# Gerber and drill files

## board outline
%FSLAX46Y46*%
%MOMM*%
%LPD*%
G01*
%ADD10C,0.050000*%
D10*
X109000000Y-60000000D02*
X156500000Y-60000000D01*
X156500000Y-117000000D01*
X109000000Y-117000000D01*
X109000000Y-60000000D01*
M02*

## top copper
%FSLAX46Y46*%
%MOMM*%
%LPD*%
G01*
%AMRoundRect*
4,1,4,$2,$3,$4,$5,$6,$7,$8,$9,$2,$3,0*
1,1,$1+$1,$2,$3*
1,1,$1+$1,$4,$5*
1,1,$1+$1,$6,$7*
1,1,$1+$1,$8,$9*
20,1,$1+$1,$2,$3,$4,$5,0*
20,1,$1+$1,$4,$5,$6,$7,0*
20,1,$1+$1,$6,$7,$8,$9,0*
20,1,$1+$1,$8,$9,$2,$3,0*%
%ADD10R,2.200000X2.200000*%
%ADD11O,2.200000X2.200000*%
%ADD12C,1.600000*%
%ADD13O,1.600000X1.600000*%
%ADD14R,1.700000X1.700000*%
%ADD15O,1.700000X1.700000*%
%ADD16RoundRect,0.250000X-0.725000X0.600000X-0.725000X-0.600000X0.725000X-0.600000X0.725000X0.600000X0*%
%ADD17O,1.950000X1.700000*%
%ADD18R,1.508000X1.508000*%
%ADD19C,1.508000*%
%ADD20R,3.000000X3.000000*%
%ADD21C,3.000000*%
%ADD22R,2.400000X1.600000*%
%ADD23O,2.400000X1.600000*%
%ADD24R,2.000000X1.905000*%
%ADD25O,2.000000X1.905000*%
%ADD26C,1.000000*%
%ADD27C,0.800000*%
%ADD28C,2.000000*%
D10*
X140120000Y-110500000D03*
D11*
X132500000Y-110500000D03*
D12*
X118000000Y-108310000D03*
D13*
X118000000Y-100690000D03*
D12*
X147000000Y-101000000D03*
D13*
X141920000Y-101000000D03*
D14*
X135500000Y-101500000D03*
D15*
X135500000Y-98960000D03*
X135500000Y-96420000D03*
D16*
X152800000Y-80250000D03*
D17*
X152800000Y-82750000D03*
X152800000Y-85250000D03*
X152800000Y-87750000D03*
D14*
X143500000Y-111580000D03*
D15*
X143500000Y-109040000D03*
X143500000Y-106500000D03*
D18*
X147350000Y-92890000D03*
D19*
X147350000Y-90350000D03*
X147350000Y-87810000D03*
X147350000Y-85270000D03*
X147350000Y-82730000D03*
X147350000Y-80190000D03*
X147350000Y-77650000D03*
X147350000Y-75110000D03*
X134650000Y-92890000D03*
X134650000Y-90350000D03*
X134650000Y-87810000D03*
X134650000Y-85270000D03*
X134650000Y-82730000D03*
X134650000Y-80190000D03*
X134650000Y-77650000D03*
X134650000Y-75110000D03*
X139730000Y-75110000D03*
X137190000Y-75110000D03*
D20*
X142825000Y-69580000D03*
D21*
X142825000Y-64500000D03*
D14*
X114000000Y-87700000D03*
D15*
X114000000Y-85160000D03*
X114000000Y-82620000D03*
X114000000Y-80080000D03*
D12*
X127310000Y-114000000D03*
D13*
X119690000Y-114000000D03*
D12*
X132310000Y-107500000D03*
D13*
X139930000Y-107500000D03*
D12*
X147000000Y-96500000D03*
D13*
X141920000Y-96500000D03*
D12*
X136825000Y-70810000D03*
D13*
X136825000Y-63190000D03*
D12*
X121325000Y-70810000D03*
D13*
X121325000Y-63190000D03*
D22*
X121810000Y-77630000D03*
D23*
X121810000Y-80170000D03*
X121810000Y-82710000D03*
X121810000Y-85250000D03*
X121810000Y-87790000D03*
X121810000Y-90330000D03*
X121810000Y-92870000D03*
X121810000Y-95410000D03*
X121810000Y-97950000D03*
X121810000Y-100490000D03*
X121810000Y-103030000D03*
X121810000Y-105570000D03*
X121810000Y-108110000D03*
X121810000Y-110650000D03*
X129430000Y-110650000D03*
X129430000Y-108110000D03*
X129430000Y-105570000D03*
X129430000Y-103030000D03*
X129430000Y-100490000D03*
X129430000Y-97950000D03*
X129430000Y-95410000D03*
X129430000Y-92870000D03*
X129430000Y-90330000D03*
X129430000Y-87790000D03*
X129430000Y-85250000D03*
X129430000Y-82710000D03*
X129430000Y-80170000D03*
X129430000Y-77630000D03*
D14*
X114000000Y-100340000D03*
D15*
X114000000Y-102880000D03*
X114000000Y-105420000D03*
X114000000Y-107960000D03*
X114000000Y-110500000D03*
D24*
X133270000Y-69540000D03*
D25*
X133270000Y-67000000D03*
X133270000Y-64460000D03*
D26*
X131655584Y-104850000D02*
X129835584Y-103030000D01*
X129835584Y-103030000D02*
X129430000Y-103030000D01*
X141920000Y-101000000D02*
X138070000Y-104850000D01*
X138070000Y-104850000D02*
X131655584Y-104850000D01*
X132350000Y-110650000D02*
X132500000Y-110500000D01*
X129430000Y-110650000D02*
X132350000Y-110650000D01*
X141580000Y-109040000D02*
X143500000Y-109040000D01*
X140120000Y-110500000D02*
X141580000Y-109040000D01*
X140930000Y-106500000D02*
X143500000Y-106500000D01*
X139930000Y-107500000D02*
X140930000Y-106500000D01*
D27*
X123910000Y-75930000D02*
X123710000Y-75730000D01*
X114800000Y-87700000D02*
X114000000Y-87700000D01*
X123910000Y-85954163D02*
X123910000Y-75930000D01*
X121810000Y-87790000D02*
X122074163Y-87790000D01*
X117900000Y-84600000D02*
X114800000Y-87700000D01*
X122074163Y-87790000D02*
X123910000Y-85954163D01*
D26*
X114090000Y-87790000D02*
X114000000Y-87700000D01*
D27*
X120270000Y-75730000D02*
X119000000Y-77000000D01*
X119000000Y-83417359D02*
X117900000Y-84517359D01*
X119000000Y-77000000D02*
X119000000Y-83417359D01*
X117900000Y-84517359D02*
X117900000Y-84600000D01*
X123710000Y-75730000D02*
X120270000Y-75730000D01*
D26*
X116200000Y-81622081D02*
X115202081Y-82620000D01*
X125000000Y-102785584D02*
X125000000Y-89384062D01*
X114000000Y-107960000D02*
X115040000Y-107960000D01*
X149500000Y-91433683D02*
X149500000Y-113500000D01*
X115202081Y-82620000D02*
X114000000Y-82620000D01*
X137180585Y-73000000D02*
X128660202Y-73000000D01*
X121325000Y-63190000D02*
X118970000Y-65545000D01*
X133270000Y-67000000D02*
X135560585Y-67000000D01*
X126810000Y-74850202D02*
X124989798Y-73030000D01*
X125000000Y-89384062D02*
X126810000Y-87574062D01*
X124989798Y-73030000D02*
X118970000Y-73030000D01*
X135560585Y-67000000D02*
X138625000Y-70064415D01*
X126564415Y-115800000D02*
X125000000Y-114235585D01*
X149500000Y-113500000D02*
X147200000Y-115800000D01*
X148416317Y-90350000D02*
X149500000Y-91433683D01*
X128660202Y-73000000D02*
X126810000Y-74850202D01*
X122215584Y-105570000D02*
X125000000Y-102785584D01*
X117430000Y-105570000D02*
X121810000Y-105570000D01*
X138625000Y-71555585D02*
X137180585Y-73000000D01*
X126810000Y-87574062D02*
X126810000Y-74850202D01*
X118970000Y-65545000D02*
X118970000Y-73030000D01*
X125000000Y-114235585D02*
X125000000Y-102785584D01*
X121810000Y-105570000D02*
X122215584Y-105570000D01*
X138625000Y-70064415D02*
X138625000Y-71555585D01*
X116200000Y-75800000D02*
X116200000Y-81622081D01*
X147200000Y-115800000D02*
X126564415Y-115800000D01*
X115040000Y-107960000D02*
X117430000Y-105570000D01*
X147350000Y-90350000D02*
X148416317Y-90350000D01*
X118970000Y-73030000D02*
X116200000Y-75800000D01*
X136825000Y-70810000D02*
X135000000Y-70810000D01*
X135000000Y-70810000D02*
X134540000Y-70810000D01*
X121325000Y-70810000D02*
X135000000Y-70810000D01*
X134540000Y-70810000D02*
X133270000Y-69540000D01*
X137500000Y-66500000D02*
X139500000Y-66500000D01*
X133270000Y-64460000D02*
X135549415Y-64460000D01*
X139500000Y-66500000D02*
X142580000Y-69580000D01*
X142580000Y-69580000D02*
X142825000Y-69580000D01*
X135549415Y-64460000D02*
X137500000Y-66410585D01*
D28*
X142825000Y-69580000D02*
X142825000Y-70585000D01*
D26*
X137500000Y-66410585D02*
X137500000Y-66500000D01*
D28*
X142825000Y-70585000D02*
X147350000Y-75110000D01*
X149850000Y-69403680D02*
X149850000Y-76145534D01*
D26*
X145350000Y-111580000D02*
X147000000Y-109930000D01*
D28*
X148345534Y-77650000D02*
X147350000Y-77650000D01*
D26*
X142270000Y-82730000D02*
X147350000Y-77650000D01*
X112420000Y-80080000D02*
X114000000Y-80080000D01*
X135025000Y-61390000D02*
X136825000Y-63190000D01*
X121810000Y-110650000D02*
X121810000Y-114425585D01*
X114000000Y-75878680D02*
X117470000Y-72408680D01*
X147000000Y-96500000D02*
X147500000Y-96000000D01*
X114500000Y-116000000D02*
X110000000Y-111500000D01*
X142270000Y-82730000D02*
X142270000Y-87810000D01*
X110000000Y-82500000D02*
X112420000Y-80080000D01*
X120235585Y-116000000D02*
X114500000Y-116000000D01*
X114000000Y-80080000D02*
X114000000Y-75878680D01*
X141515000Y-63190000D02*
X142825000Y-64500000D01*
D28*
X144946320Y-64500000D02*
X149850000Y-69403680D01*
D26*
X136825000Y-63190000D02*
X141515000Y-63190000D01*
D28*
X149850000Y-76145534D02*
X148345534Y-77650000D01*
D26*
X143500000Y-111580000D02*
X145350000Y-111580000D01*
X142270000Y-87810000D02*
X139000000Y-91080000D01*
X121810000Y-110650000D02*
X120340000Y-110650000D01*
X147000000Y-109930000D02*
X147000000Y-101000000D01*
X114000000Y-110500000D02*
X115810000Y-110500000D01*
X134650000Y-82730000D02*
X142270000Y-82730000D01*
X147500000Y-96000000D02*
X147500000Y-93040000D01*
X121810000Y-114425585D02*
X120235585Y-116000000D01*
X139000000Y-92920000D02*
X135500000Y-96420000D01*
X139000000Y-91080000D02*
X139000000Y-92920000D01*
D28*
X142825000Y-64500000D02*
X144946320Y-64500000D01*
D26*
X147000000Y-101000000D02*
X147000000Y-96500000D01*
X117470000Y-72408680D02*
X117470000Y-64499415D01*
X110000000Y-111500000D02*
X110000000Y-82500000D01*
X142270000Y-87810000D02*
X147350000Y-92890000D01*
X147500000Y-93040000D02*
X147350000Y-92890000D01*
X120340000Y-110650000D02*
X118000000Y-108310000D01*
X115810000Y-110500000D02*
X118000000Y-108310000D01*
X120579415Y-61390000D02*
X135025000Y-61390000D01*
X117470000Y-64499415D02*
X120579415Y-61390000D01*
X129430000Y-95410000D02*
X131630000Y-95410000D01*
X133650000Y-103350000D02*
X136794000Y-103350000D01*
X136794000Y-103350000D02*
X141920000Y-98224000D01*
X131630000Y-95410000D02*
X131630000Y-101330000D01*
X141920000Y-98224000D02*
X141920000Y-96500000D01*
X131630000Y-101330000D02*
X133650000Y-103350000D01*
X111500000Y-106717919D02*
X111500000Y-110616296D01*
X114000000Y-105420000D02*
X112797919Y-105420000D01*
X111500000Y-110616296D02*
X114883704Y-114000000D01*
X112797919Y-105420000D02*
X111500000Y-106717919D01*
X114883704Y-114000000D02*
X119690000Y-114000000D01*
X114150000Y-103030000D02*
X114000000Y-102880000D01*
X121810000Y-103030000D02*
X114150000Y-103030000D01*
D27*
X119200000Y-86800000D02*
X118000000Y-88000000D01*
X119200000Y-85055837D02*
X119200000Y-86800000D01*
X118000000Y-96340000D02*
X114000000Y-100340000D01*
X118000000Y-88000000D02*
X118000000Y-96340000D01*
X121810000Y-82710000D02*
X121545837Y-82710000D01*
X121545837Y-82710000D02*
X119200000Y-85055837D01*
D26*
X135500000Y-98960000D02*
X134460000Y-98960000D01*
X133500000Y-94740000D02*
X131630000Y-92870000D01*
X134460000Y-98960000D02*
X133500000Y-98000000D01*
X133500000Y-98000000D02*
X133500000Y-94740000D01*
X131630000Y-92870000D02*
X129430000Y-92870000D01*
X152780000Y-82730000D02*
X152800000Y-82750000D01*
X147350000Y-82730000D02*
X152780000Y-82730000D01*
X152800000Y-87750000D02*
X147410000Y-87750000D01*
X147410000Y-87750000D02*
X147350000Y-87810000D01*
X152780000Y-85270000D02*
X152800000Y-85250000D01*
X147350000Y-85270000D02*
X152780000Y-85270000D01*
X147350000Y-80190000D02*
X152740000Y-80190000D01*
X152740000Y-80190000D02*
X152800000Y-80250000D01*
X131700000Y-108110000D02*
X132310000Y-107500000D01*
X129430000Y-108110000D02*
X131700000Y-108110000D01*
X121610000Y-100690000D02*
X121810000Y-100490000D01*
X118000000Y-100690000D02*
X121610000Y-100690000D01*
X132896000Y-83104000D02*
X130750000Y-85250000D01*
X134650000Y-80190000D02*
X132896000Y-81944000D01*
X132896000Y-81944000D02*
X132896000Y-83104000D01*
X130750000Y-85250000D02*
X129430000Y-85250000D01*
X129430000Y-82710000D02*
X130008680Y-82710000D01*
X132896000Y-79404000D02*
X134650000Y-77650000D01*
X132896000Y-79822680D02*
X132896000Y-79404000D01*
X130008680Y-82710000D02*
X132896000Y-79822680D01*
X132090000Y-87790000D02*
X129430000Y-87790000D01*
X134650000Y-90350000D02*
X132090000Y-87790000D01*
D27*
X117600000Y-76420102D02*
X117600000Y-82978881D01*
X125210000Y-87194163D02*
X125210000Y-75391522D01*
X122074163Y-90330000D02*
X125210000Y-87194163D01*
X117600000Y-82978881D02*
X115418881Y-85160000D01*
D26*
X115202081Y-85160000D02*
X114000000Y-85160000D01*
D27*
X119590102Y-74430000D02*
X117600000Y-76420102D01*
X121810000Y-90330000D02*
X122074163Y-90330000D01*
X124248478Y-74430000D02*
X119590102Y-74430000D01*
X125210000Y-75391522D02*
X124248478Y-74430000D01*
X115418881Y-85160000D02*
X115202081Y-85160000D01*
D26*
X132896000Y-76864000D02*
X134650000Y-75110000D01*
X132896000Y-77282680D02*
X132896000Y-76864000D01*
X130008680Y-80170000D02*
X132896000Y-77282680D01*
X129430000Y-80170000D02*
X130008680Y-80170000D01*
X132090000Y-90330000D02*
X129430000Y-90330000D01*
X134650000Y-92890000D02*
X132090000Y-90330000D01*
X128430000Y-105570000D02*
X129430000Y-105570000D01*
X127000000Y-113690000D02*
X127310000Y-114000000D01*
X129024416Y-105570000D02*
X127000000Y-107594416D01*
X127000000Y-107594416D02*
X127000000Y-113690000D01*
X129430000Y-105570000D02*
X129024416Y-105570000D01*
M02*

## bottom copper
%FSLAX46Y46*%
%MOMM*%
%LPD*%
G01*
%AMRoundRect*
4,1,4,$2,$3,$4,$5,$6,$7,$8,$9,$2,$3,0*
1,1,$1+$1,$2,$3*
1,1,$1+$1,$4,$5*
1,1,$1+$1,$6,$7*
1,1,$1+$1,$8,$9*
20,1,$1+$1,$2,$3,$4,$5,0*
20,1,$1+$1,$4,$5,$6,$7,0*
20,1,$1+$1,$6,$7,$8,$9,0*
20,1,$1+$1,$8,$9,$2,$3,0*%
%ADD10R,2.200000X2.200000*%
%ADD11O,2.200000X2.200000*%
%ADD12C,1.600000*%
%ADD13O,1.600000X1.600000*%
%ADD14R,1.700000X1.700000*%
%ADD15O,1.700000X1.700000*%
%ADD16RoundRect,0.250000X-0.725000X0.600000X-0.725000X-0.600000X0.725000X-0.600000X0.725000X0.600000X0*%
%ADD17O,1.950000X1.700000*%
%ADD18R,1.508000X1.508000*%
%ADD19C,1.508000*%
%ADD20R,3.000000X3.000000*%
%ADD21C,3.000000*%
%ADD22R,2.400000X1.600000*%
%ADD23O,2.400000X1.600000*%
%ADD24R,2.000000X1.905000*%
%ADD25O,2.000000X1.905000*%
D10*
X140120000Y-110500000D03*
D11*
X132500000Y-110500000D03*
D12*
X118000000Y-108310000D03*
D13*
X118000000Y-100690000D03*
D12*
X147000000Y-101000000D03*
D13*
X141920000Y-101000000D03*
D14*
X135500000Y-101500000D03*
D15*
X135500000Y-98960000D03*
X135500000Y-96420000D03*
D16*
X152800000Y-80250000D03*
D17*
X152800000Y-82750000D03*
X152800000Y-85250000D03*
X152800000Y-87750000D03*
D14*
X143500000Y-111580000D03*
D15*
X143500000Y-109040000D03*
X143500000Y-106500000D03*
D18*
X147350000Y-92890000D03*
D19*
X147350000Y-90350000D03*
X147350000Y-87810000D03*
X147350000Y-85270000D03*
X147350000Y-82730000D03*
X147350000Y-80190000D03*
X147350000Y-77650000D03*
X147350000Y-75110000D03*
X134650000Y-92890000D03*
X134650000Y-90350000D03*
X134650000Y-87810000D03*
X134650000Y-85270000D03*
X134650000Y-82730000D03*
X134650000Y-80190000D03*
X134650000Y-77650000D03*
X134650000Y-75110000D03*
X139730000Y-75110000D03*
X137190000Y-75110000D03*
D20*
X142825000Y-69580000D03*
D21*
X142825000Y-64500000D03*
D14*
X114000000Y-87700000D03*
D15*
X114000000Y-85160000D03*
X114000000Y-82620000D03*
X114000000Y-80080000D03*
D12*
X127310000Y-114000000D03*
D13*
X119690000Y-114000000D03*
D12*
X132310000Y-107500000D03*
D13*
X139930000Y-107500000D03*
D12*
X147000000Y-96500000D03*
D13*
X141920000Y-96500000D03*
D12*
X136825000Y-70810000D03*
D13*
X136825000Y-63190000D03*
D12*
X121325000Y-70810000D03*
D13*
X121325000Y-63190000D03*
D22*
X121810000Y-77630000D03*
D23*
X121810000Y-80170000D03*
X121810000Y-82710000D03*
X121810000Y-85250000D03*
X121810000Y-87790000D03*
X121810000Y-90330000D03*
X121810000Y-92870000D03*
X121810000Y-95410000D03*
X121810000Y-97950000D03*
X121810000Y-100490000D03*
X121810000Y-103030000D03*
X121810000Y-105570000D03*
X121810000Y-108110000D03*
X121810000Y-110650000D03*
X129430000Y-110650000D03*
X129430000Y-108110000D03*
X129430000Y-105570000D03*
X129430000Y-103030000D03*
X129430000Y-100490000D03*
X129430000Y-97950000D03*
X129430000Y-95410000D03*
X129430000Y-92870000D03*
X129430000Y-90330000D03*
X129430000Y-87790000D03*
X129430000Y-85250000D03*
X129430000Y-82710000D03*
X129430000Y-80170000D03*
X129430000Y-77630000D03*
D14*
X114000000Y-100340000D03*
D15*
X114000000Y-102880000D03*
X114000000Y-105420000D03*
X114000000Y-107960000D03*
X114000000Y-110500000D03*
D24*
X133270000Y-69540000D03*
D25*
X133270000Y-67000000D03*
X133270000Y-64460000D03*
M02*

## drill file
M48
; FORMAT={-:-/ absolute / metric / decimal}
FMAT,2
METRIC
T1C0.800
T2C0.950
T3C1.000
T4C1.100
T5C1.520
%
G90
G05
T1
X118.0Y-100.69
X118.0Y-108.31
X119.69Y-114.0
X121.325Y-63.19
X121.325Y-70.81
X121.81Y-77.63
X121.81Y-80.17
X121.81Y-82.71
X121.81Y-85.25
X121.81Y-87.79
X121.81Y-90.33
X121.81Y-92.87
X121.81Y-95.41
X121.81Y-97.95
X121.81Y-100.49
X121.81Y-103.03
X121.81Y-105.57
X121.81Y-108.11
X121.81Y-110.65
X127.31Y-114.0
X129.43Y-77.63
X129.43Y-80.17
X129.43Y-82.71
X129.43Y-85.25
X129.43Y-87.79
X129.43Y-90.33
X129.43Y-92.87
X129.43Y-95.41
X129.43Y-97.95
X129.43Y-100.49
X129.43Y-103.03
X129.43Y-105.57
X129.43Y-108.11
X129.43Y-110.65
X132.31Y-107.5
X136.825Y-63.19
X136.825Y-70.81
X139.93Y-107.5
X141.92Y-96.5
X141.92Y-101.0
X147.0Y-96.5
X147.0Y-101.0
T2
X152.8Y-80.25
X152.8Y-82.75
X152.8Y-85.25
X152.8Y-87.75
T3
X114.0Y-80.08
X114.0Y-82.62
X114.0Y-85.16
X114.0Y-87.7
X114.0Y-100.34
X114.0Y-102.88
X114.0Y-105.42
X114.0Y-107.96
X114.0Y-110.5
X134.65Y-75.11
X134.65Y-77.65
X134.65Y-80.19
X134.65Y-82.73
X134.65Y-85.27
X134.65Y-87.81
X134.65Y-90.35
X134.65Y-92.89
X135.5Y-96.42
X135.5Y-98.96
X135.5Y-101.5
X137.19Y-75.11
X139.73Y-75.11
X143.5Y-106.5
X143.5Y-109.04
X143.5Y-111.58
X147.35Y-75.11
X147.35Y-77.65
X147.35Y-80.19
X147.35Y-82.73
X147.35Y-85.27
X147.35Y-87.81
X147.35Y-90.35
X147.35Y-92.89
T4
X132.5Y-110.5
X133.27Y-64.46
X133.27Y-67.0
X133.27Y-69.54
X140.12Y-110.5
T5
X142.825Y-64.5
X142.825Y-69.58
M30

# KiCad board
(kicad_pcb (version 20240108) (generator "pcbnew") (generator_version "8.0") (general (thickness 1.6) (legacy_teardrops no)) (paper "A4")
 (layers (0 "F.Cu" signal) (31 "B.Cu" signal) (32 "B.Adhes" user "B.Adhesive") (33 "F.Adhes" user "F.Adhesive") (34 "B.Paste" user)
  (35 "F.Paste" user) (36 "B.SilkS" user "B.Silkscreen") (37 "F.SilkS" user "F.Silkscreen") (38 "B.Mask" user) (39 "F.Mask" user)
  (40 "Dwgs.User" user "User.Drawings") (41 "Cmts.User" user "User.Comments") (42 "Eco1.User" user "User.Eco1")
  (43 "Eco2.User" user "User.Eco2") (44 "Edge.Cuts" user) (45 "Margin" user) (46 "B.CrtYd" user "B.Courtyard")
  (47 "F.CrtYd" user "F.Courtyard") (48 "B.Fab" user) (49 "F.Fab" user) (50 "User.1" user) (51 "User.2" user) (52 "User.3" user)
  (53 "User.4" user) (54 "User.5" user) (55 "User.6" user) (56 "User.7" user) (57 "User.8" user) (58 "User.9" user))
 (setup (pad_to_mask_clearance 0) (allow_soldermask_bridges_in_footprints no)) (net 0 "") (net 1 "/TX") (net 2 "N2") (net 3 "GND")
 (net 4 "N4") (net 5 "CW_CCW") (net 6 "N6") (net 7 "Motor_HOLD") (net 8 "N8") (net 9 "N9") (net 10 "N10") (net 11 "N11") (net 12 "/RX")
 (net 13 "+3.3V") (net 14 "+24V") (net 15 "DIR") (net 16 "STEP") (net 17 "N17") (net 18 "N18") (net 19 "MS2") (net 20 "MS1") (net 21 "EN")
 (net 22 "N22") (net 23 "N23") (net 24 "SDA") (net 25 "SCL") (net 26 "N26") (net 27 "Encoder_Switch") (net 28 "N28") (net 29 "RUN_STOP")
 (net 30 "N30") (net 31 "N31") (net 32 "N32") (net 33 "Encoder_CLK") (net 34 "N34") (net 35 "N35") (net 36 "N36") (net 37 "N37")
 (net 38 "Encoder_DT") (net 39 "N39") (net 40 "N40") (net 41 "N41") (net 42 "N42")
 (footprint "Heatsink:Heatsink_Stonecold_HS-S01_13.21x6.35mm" (layer "F.Cu") (at 129.5 67 -90)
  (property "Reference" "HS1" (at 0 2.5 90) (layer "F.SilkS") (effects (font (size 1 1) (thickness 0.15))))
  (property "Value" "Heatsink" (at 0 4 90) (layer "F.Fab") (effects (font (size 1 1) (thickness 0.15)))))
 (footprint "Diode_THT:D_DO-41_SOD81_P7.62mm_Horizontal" (layer "F.Cu") (at 140.12 110.5 180)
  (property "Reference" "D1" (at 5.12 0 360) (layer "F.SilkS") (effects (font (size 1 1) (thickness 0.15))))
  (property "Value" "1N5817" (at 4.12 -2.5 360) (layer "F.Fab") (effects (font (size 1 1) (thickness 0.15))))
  (pad "1" thru_hole rect (at 0 0 180) (size 2.2 2.2) (drill 1.1) (layers "*.Cu" "*.Mask") (remove_unused_layers no) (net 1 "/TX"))
  (pad "2" thru_hole oval (at 7.62 0 180) (size 2.2 2.2) (drill 1.1) (layers "*.Cu" "*.Mask") (remove_unused_layers no) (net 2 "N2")))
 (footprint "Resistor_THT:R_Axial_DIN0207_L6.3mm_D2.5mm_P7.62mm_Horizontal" (layer "F.Cu") (at 118 108.31 90)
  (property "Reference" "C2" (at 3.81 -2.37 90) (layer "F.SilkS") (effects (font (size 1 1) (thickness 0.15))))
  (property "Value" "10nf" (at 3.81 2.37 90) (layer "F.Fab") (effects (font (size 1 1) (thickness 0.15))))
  (pad "1" thru_hole circle (at 0 0 90) (size 1.6 1.6) (drill 0.8) (layers "*.Cu" "*.Mask") (remove_unused_layers no) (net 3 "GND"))
  (pad "2" thru_hole oval (at 7.62 0 90) (size 1.6 1.6) (drill 0.8) (layers "*.Cu" "*.Mask") (remove_unused_layers no) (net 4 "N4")))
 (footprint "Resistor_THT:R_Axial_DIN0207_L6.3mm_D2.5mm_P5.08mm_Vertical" (layer "F.Cu") (at 147 101 180)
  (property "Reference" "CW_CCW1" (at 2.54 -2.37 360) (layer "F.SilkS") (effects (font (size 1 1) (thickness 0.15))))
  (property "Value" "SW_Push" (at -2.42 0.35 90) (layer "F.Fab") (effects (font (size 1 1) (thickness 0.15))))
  (pad "1" thru_hole circle (at 0 0 180) (size 1.6 1.6) (drill 0.8) (layers "*.Cu" "*.Mask") (remove_unused_layers no) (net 3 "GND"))
  (pad "2" thru_hole oval (at 5.08 0 180) (size 1.6 1.6) (drill 0.8) (layers "*.Cu" "*.Mask") (remove_unused_layers no) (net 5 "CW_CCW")))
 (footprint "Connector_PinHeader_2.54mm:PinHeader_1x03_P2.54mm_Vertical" (layer "F.Cu") (at 135.5 101.5 180)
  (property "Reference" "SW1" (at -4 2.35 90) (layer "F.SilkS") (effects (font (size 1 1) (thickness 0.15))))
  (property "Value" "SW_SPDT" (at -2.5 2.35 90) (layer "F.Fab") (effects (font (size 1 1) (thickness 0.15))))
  (pad "1" thru_hole rect (at 0 0 180) (size 1.7 1.7) (drill 1) (layers "*.Cu" "*.Mask") (remove_unused_layers no) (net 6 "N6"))
  (pad "2" thru_hole oval (at 0 2.54 180) (size 1.7 1.7) (drill 1) (layers "*.Cu" "*.Mask") (remove_unused_layers no) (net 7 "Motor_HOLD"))
  (pad "3" thru_hole oval (at 0 5.08 180) (size 1.7 1.7) (drill 1) (layers "*.Cu" "*.Mask") (remove_unused_layers no) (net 3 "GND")))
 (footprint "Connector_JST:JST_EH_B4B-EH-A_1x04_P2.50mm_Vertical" (layer "F.Cu") (at 152.8 80.25 -90)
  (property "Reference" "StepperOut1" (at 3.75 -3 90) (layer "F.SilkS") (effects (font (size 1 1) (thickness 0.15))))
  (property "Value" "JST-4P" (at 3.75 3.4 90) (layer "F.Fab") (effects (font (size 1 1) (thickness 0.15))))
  (pad "1" thru_hole roundrect (at 0 0 270) (size 1.7 1.95) (drill 0.95) (layers "*.Cu" "*.Mask") (remove_unused_layers no)
   (roundrect_rratio 0.147059) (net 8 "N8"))
  (pad "2" thru_hole oval (at 2.5 0 270) (size 1.7 1.95) (drill 0.95) (layers "*.Cu" "*.Mask") (remove_unused_layers no) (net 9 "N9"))
  (pad "3" thru_hole oval (at 5 0 270) (size 1.7 1.95) (drill 0.95) (layers "*.Cu" "*.Mask") (remove_unused_layers no) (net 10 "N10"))
  (pad "4" thru_hole oval (at 7.5 0 270) (size 1.7 1.95) (drill 0.95) (layers "*.Cu" "*.Mask") (remove_unused_layers no) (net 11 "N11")))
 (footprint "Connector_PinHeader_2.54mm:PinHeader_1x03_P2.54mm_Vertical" (layer "F.Cu") (at 143.5 111.58 180)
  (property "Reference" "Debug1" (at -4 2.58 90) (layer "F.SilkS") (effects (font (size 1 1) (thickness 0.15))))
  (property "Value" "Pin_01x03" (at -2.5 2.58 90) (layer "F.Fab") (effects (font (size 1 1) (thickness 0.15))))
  (pad "1" thru_hole rect (at 0 0 180) (size 1.7 1.7) (drill 1) (layers "*.Cu" "*.Mask") (remove_unused_layers no) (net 3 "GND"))
  (pad "2" thru_hole oval (at 0 2.54 180) (size 1.7 1.7) (drill 1) (layers "*.Cu" "*.Mask") (remove_unused_layers no) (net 1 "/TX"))
  (pad "3" thru_hole oval (at 0 5.08 180) (size 1.7 1.7) (drill 1) (layers "*.Cu" "*.Mask") (remove_unused_layers no) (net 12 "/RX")))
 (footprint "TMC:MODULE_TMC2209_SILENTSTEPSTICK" (layer "F.Cu") (at 141 84 180)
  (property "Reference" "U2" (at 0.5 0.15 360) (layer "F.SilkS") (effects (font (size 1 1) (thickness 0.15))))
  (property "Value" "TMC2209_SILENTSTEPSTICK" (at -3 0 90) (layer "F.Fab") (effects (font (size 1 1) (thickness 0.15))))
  (pad "1" thru_hole rect (at -6.35 -8.89 180) (size 1.508 1.508) (drill 1) (layers "*.Cu" "*.Mask") (remove_unused_layers no) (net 3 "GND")
   (solder_mask_margin 0.102))
  (pad "2" thru_hole circle (at -6.35 -6.35 180) (size 1.508 1.508) (drill 1) (layers "*.Cu" "*.Mask") (remove_unused_layers no)
   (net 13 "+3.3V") (solder_mask_margin 0.102))
  (pad "3" thru_hole circle (at -6.35 -3.81 180) (size 1.508 1.508) (drill 1) (layers "*.Cu" "*.Mask") (remove_unused_layers no)
   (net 11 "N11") (solder_mask_margin 0.102))
  (pad "4" thru_hole circle (at -6.35 -1.27 180) (size 1.508 1.508) (drill 1) (layers "*.Cu" "*.Mask") (remove_unused_layers no)
   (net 10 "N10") (solder_mask_margin 0.102))
  (pad "5" thru_hole circle (at -6.35 1.27 180) (size 1.508 1.508) (drill 1) (layers "*.Cu" "*.Mask") (remove_unused_layers no) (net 9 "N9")
   (solder_mask_margin 0.102))
  (pad "6" thru_hole circle (at -6.35 3.81 180) (size 1.508 1.508) (drill 1) (layers "*.Cu" "*.Mask") (remove_unused_layers no) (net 8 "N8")
   (solder_mask_margin 0.102))
  (pad "7" thru_hole circle (at -6.35 6.35 180) (size 1.508 1.508) (drill 1) (layers "*.Cu" "*.Mask") (remove_unused_layers no)
   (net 3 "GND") (solder_mask_margin 0.102))
  (pad "8" thru_hole circle (at -6.35 8.89 180) (size 1.508 1.508) (drill 1) (layers "*.Cu" "*.Mask") (remove_unused_layers no)
   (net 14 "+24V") (solder_mask_margin 0.102))
  (pad "9" thru_hole circle (at 6.35 -8.89 180) (size 1.508 1.508) (drill 1) (layers "*.Cu" "*.Mask") (remove_unused_layers no)
   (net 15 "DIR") (solder_mask_margin 0.102))
  (pad "10" thru_hole circle (at 6.35 -6.35 180) (size 1.508 1.508) (drill 1) (layers "*.Cu" "*.Mask") (remove_unused_layers no)
   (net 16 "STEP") (solder_mask_margin 0.102))
  (pad "11" thru_hole circle (at 6.35 -3.81 180) (size 1.508 1.508) (drill 1) (layers "*.Cu" "*.Mask") (remove_unused_layers no)
   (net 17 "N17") (solder_mask_margin 0.102))
  (pad "12" thru_hole circle (at 6.35 -1.27 180) (size 1.508 1.508) (drill 1) (layers "*.Cu" "*.Mask") (remove_unused_layers no)
   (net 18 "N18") (solder_mask_margin 0.102))
  (pad "13" thru_hole circle (at 6.35 1.27 180) (size 1.508 1.508) (drill 1) (layers "*.Cu" "*.Mask") (remove_unused_layers no)
   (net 3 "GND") (solder_mask_margin 0.102))
  (pad "14" thru_hole circle (at 6.35 3.81 180) (size 1.508 1.508) (drill 1) (layers "*.Cu" "*.Mask") (remove_unused_layers no)
   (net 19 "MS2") (solder_mask_margin 0.102))
  (pad "15" thru_hole circle (at 6.35 6.35 180) (size 1.508 1.508) (drill 1) (layers "*.Cu" "*.Mask") (remove_unused_layers no)
   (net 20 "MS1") (solder_mask_margin 0.102))
  (pad "16" thru_hole circle (at 6.35 8.89 180) (size 1.508 1.508) (drill 1) (layers "*.Cu" "*.Mask") (remove_unused_layers no)
   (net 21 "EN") (solder_mask_margin 0.102))
  (pad "17" thru_hole circle (at 1.27 8.89 180) (size 1.508 1.508) (drill 1) (layers "*.Cu" "*.Mask") (remove_unused_layers no)
   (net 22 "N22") (solder_mask_margin 0.102))
  (pad "18" thru_hole circle (at 3.81 8.89 180) (size 1.508 1.508) (drill 1) (layers "*.Cu" "*.Mask") (remove_unused_layers no)
   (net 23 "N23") (solder_mask_margin 0.102)))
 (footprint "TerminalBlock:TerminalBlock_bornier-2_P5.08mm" (layer "F.Cu") (at 142.825 69.58 90)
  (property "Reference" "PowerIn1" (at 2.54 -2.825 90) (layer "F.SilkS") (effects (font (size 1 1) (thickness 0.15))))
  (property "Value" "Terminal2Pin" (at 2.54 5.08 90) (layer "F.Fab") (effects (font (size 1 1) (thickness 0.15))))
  (pad "1" thru_hole rect (at 0 0 90) (size 3 3) (drill 1.52) (layers "*.Cu" "*.Mask") (remove_unused_layers no) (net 14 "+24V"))
  (pad "2" thru_hole circle (at 5.08 0 90) (size 3 3) (drill 1.52) (layers "*.Cu" "*.Mask") (remove_unused_layers no) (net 3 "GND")))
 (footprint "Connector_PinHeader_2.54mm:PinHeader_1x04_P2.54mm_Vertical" (layer "F.Cu") (at 114 87.7 180)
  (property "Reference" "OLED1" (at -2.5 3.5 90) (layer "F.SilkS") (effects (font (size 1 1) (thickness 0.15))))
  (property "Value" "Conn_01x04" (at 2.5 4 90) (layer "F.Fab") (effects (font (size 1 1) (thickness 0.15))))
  (pad "1" thru_hole rect (at 0 0 180) (size 1.7 1.7) (drill 1) (layers "*.Cu" "*.Mask") (remove_unused_layers no) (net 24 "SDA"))
  (pad "2" thru_hole oval (at 0 2.54 180) (size 1.7 1.7) (drill 1) (layers "*.Cu" "*.Mask") (remove_unused_layers no) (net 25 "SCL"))
  (pad "3" thru_hole oval (at 0 5.08 180) (size 1.7 1.7) (drill 1) (layers "*.Cu" "*.Mask") (remove_unused_layers no) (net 13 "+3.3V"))
  (pad "4" thru_hole oval (at 0 7.62 180) (size 1.7 1.7) (drill 1) (layers "*.Cu" "*.Mask") (remove_unused_layers no) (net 3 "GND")))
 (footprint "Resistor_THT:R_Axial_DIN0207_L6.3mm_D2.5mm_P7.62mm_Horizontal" (layer "F.Cu") (at 127.31 114 180)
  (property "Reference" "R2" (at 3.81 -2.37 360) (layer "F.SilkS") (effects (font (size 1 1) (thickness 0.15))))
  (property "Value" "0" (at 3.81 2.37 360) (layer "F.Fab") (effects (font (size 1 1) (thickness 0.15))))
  (pad "1" thru_hole circle (at 0 0 180) (size 1.6 1.6) (drill 0.8) (layers "*.Cu" "*.Mask") (remove_unused_layers no) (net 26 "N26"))
  (pad "2" thru_hole oval (at 7.62 0 180) (size 1.6 1.6) (drill 0.8) (layers "*.Cu" "*.Mask") (remove_unused_layers no)
   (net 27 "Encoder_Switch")))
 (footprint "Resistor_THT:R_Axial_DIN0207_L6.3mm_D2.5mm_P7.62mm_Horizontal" (layer "F.Cu") (at 132.31 107.5)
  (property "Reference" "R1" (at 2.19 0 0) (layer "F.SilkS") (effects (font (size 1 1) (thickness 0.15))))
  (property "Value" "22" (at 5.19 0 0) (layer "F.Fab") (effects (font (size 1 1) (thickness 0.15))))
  (pad "1" thru_hole circle (at 0 0) (size 1.6 1.6) (drill 0.8) (layers "*.Cu" "*.Mask") (remove_unused_layers no) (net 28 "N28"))
  (pad "2" thru_hole oval (at 7.62 0) (size 1.6 1.6) (drill 0.8) (layers "*.Cu" "*.Mask") (remove_unused_layers no) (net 12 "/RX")))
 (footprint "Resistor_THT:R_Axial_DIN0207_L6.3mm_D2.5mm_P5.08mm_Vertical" (layer "F.Cu") (at 147 96.5 180)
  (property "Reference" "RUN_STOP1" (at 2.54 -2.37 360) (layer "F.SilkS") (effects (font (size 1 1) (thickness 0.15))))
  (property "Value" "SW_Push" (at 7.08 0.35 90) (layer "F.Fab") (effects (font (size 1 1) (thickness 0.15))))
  (pad "1" thru_hole circle (at 0 0 180) (size 1.6 1.6) (drill 0.8) (layers "*.Cu" "*.Mask") (remove_unused_layers no) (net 3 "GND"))
  (pad "2" thru_hole oval (at 5.08 0 180) (size 1.6 1.6) (drill 0.8) (layers "*.Cu" "*.Mask") (remove_unused_layers no) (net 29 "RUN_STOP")))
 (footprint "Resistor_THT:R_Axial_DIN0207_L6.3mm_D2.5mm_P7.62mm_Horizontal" (layer "F.Cu") (at 136.825 70.81 90)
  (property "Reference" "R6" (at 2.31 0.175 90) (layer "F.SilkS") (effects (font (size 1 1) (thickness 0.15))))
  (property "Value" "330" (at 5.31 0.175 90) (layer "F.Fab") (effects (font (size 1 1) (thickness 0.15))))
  (pad "1" thru_hole circle (at 0 0 90) (size 1.6 1.6) (drill 0.8) (layers "*.Cu" "*.Mask") (remove_unused_layers no) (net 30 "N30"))
  (pad "2" thru_hole oval (at 7.62 0 90) (size 1.6 1.6) (drill 0.8) (layers "*.Cu" "*.Mask") (remove_unused_layers no) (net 3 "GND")))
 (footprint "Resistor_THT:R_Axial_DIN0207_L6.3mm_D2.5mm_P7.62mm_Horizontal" (layer "F.Cu") (at 121.325 70.81 90)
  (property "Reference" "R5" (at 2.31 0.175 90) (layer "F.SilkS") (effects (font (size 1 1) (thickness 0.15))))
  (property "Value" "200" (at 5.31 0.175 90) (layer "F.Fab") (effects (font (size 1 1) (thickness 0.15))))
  (pad "1" thru_hole circle (at 0 0 90) (size 1.6 1.6) (drill 0.8) (layers "*.Cu" "*.Mask") (remove_unused_layers no) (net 30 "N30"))
  (pad "2" thru_hole oval (at 7.62 0 90) (size 1.6 1.6) (drill 0.8) (layers "*.Cu" "*.Mask") (remove_unused_layers no) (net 13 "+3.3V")))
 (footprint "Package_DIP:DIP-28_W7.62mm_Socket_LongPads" (layer "F.Cu") (at 121.81 77.63)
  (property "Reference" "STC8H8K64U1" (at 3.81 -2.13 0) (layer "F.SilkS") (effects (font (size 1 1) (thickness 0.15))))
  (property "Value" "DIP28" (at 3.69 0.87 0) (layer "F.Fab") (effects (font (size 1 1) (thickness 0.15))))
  (pad "1" thru_hole rect (at 0 0) (size 2.4 1.6) (drill 0.8) (layers "*.Cu" "*.Mask") (remove_unused_layers no) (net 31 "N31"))
  (pad "2" thru_hole oval (at 0 2.54) (size 2.4 1.6) (drill 0.8) (layers "*.Cu" "*.Mask") (remove_unused_layers no) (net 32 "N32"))
  (pad "3" thru_hole oval (at 0 5.08) (size 2.4 1.6) (drill 0.8) (layers "*.Cu" "*.Mask") (remove_unused_layers no) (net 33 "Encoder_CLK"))
  (pad "4" thru_hole oval (at 0 7.62) (size 2.4 1.6) (drill 0.8) (layers "*.Cu" "*.Mask") (remove_unused_layers no) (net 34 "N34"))
  (pad "5" thru_hole oval (at 0 10.16) (size 2.4 1.6) (drill 0.8) (layers "*.Cu" "*.Mask") (remove_unused_layers no) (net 24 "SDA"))
  (pad "6" thru_hole oval (at 0 12.7) (size 2.4 1.6) (drill 0.8) (layers "*.Cu" "*.Mask") (remove_unused_layers no) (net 25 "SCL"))
  (pad "7" thru_hole oval (at 0 15.24) (size 2.4 1.6) (drill 0.8) (layers "*.Cu" "*.Mask") (remove_unused_layers no) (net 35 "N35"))
  (pad "8" thru_hole oval (at 0 17.78) (size 2.4 1.6) (drill 0.8) (layers "*.Cu" "*.Mask") (remove_unused_layers no) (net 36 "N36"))
  (pad "9" thru_hole oval (at 0 20.32) (size 2.4 1.6) (drill 0.8) (layers "*.Cu" "*.Mask") (remove_unused_layers no) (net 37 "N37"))
  (pad "10" thru_hole oval (at 0 22.86) (size 2.4 1.6) (drill 0.8) (layers "*.Cu" "*.Mask") (remove_unused_layers no) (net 4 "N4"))
  (pad "11" thru_hole oval (at 0 25.4) (size 2.4 1.6) (drill 0.8) (layers "*.Cu" "*.Mask") (remove_unused_layers no) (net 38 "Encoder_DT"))
  (pad "12" thru_hole oval (at 0 27.94) (size 2.4 1.6) (drill 0.8) (layers "*.Cu" "*.Mask") (remove_unused_layers no) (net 13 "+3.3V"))
  (pad "13" thru_hole oval (at 0 30.48) (size 2.4 1.6) (drill 0.8) (layers "*.Cu" "*.Mask") (remove_unused_layers no) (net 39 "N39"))
  (pad "14" thru_hole oval (at 0 33.02) (size 2.4 1.6) (drill 0.8) (layers "*.Cu" "*.Mask") (remove_unused_layers no) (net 3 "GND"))
  (pad "15" thru_hole oval (at 7.62 33.02) (size 2.4 1.6) (drill 0.8) (layers "*.Cu" "*.Mask") (remove_unused_layers no) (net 2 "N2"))
  (pad "16" thru_hole oval (at 7.62 30.48) (size 2.4 1.6) (drill 0.8) (layers "*.Cu" "*.Mask") (remove_unused_layers no) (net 28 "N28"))
  (pad "17" thru_hole oval (at 7.62 27.94) (size 2.4 1.6) (drill 0.8) (layers "*.Cu" "*.Mask") (remove_unused_layers no) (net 26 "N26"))
  (pad "18" thru_hole oval (at 7.62 25.4) (size 2.4 1.6) (drill 0.8) (layers "*.Cu" "*.Mask") (remove_unused_layers no) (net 5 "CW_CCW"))
  (pad "19" thru_hole oval (at 7.62 22.86) (size 2.4 1.6) (drill 0.8) (layers "*.Cu" "*.Mask") (remove_unused_layers no) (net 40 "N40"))
  (pad "20" thru_hole oval (at 7.62 20.32) (size 2.4 1.6) (drill 0.8) (layers "*.Cu" "*.Mask") (remove_unused_layers no) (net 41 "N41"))
  (pad "21" thru_hole oval (at 7.62 17.78) (size 2.4 1.6) (drill 0.8) (layers "*.Cu" "*.Mask") (remove_unused_layers no) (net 29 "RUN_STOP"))
  (pad "22" thru_hole oval (at 7.62 15.24) (size 2.4 1.6) (drill 0.8) (layers "*.Cu" "*.Mask") (remove_unused_layers no)
   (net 7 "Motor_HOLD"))
  (pad "23" thru_hole oval (at 7.62 12.7) (size 2.4 1.6) (drill 0.8) (layers "*.Cu" "*.Mask") (remove_unused_layers no) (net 15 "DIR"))
  (pad "24" thru_hole oval (at 7.62 10.16) (size 2.4 1.6) (drill 0.8) (layers "*.Cu" "*.Mask") (remove_unused_layers no) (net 16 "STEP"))
  (pad "25" thru_hole oval (at 7.62 7.62) (size 2.4 1.6) (drill 0.8) (layers "*.Cu" "*.Mask") (remove_unused_layers no) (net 19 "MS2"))
  (pad "26" thru_hole oval (at 7.62 5.08) (size 2.4 1.6) (drill 0.8) (layers "*.Cu" "*.Mask") (remove_unused_layers no) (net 20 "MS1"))
  (pad "27" thru_hole oval (at 7.62 2.54) (size 2.4 1.6) (drill 0.8) (layers "*.Cu" "*.Mask") (remove_unused_layers no) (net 21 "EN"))
  (pad "28" thru_hole oval (at 7.62 0) (size 2.4 1.6) (drill 0.8) (layers "*.Cu" "*.Mask") (remove_unused_layers no) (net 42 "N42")))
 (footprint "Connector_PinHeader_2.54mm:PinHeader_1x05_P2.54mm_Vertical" (layer "F.Cu") (at 114 100.34)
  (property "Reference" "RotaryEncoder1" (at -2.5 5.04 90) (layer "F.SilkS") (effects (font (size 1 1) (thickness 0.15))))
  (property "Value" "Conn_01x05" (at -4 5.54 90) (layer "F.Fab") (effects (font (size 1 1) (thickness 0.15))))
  (pad "1" thru_hole rect (at 0 0) (size 1.7 1.7) (drill 1) (layers "*.Cu" "*.Mask") (remove_unused_layers no) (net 33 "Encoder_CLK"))
  (pad "2" thru_hole oval (at 0 2.54) (size 1.7 1.7) (drill 1) (layers "*.Cu" "*.Mask") (remove_unused_layers no) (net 38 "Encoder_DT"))
  (pad "3" thru_hole oval (at 0 5.08) (size 1.7 1.7) (drill 1) (layers "*.Cu" "*.Mask") (remove_unused_layers no) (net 27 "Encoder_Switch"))
  (pad "4" thru_hole oval (at 0 7.62) (size 1.7 1.7) (drill 1) (layers "*.Cu" "*.Mask") (remove_unused_layers no) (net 13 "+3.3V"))
  (pad "5" thru_hole oval (at 0 10.16) (size 1.7 1.7) (drill 1) (layers "*.Cu" "*.Mask") (remove_unused_layers no) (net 3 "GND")))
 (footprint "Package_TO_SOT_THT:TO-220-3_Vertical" (layer "F.Cu") (at 133.27 69.54 90)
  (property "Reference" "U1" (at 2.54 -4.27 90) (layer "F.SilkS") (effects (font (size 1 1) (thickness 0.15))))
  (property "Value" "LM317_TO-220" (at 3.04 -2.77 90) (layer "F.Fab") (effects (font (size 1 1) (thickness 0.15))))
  (pad "1" thru_hole rect (at 0 0 90) (size 1.905 2) (drill 1.1) (layers "*.Cu" "*.Mask") (remove_unused_layers no) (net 30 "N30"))
  (pad "2" thru_hole oval (at 2.54 0 90) (size 1.905 2) (drill 1.1) (layers "*.Cu" "*.Mask") (remove_unused_layers no) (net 13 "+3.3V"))
  (pad "3" thru_hole oval (at 5.08 0 90) (size 1.905 2) (drill 1.1) (layers "*.Cu" "*.Mask") (remove_unused_layers no) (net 14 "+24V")))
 (gr_rect (start 109 60) (end 156.5 117) (stroke (width 0.05) (type default)) (fill none) (layer "Edge.Cuts"))
 (segment (start 131.655584 104.85) (end 129.835584 103.03) (width 1) (layer "F.Cu") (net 5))
 (segment (start 129.835584 103.03) (end 129.43 103.03) (width 1) (layer "F.Cu") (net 5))
 (segment (start 141.92 101) (end 138.07 104.85) (width 1) (layer "F.Cu") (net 5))
 (segment (start 138.07 104.85) (end 131.655584 104.85) (width 1) (layer "F.Cu") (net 5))
 (segment (start 132.35 110.65) (end 132.5 110.5) (width 1) (layer "F.Cu") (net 2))
 (segment (start 129.43 110.65) (end 132.35 110.65) (width 1) (layer "F.Cu") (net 2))
 (segment (start 141.58 109.04) (end 143.5 109.04) (width 1) (layer "F.Cu") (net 1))
 (segment (start 140.12 110.5) (end 141.58 109.04) (width 1) (layer "F.Cu") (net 1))
 (segment (start 140.93 106.5) (end 143.5 106.5) (width 1) (layer "F.Cu") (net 12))
 (segment (start 139.93 107.5) (end 140.93 106.5) (width 1) (layer "F.Cu") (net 12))
 (segment (start 123.91 75.93) (end 123.71 75.73) (width 0.8) (layer "F.Cu") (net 24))
 (segment (start 114.8 87.7) (end 114 87.7) (width 0.8) (layer "F.Cu") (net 24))
 (segment (start 123.91 85.954163) (end 123.91 75.93) (width 0.8) (layer "F.Cu") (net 24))
 (segment (start 121.81 87.79) (end 122.074163 87.79) (width 0.8) (layer "F.Cu") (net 24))
 (segment (start 117.9 84.6) (end 114.8 87.7) (width 0.8) (layer "F.Cu") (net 24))
 (segment (start 122.074163 87.79) (end 123.91 85.954163) (width 0.8) (layer "F.Cu") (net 24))
 (segment (start 114.09 87.79) (end 114 87.7) (width 1) (layer "F.Cu") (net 24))
 (segment (start 120.27 75.73) (end 119 77) (width 0.8) (layer "F.Cu") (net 24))
 (segment (start 119 83.417359) (end 117.9 84.517359) (width 0.8) (layer "F.Cu") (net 24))
 (segment (start 119 77) (end 119 83.417359) (width 0.8) (layer "F.Cu") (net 24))
 (segment (start 117.9 84.517359) (end 117.9 84.6) (width 0.8) (layer "F.Cu") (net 24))
 (segment (start 123.71 75.73) (end 120.27 75.73) (width 0.8) (layer "F.Cu") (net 24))
 (segment (start 116.2 81.622081) (end 115.202081 82.62) (width 1) (layer "F.Cu") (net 13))
 (segment (start 125 102.785584) (end 125 89.384062) (width 1) (layer "F.Cu") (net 13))
 (segment (start 114 107.96) (end 115.04 107.96) (width 1) (layer "F.Cu") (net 13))
 (segment (start 149.5 91.433683) (end 149.5 113.5) (width 1) (layer "F.Cu") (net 13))
 (segment (start 115.202081 82.62) (end 114 82.62) (width 1) (layer "F.Cu") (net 13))
 (segment (start 137.180585 73) (end 128.660202 73) (width 1) (layer "F.Cu") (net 13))
 (segment (start 121.325 63.19) (end 118.97 65.545) (width 1) (layer "F.Cu") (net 13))
 (segment (start 133.27 67) (end 135.560585 67) (width 1) (layer "F.Cu") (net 13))
 (segment (start 126.81 74.850202) (end 124.989798 73.03) (width 1) (layer "F.Cu") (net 13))
 (segment (start 125 89.384062) (end 126.81 87.574062) (width 1) (layer "F.Cu") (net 13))
 (segment (start 124.989798 73.03) (end 118.97 73.03) (width 1) (layer "F.Cu") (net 13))
 (segment (start 135.560585 67) (end 138.625 70.064415) (width 1) (layer "F.Cu") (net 13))
 (segment (start 126.564415 115.8) (end 125 114.235585) (width 1) (layer "F.Cu") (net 13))
 (segment (start 149.5 113.5) (end 147.2 115.8) (width 1) (layer "F.Cu") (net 13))
 (segment (start 148.416317 90.35) (end 149.5 91.433683) (width 1) (layer "F.Cu") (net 13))
 (segment (start 128.660202 73) (end 126.81 74.850202) (width 1) (layer "F.Cu") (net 13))
 (segment (start 122.215584 105.57) (end 125 102.785584) (width 1) (layer "F.Cu") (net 13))
 (segment (start 117.43 105.57) (end 121.81 105.57) (width 1) (layer "F.Cu") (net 13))
 (segment (start 138.625 71.555585) (end 137.180585 73) (width 1) (layer "F.Cu") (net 13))
 (segment (start 126.81 87.574062) (end 126.81 74.850202) (width 1) (layer "F.Cu") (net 13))
 (segment (start 118.97 65.545) (end 118.97 73.03) (width 1) (layer "F.Cu") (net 13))
 (segment (start 125 114.235585) (end 125 102.785584) (width 1) (layer "F.Cu") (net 13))
 (segment (start 121.81 105.57) (end 122.215584 105.57) (width 1) (layer "F.Cu") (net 13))
 (segment (start 138.625 70.064415) (end 138.625 71.555585) (width 1) (layer "F.Cu") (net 13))
 (segment (start 116.2 75.8) (end 116.2 81.622081) (width 1) (layer "F.Cu") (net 13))
 (segment (start 147.2 115.8) (end 126.564415 115.8) (width 1) (layer "F.Cu") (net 13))
 (segment (start 115.04 107.96) (end 117.43 105.57) (width 1) (layer "F.Cu") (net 13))
 (segment (start 147.35 90.35) (end 148.416317 90.35) (width 1) (layer "F.Cu") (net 13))
 (segment (start 118.97 73.03) (end 116.2 75.8) (width 1) (layer "F.Cu") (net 13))
 (segment (start 136.825 70.81) (end 135 70.81) (width 1) (layer "F.Cu") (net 30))
 (segment (start 135 70.81) (end 134.54 70.81) (width 1) (layer "F.Cu") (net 30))
 (segment (start 121.325 70.81) (end 135 70.81) (width 1) (layer "F.Cu") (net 30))
 (segment (start 134.54 70.81) (end 133.27 69.54) (width 1) (layer "F.Cu") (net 30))
 (segment (start 137.5 66.5) (end 139.5 66.5) (width 1) (layer "F.Cu") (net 14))
 (segment (start 133.27 64.46) (end 135.549415 64.46) (width 1) (layer "F.Cu") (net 14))
 (segment (start 139.5 66.5) (end 142.58 69.58) (width 1) (layer "F.Cu") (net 14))
 (segment (start 142.58 69.58) (end 142.825 69.58) (width 1) (layer "F.Cu") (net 14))
 (segment (start 135.549415 64.46) (end 137.5 66.410585) (width 1) (layer "F.Cu") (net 14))
 (segment (start 142.825 69.58) (end 142.825 70.585) (width 2) (layer "F.Cu") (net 14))
 (segment (start 137.5 66.410585) (end 137.5 66.5) (width 1) (layer "F.Cu") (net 14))
 (segment (start 142.825 70.585) (end 147.35 75.11) (width 2) (layer "F.Cu") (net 14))
 (segment (start 149.85 69.40368) (end 149.85 76.145534) (width 2) (layer "F.Cu") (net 3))
 (segment (start 145.35 111.58) (end 147 109.93) (width 1) (layer "F.Cu") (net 3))
 (segment (start 148.345534 77.65) (end 147.35 77.65) (width 2) (layer "F.Cu") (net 3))
 (segment (start 142.27 82.73) (end 147.35 77.65) (width 1) (layer "F.Cu") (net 3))
 (segment (start 112.42 80.08) (end 114 80.08) (width 1) (layer "F.Cu") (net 3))
 (segment (start 135.025 61.39) (end 136.825 63.19) (width 1) (layer "F.Cu") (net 3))
 (segment (start 121.81 110.65) (end 121.81 114.425585) (width 1) (layer "F.Cu") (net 3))
 (segment (start 114 75.87868) (end 117.47 72.40868) (width 1) (layer "F.Cu") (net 3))
 (segment (start 147 96.5) (end 147.5 96) (width 1) (layer "F.Cu") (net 3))
 (segment (start 114.5 116) (end 110 111.5) (width 1) (layer "F.Cu") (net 3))
 (segment (start 142.27 82.73) (end 142.27 87.81) (width 1) (layer "F.Cu") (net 3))
 (segment (start 110 82.5) (end 112.42 80.08) (width 1) (layer "F.Cu") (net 3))
 (segment (start 120.235585 116) (end 114.5 116) (width 1) (layer "F.Cu") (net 3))
 (segment (start 114 80.08) (end 114 75.87868) (width 1) (layer "F.Cu") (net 3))
 (segment (start 141.515 63.19) (end 142.825 64.5) (width 1) (layer "F.Cu") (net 3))
 (segment (start 144.94632 64.5) (end 149.85 69.40368) (width 2) (layer "F.Cu") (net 3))
 (segment (start 136.825 63.19) (end 141.515 63.19) (width 1) (layer "F.Cu") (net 3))
 (segment (start 149.85 76.145534) (end 148.345534 77.65) (width 2) (layer "F.Cu") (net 3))
 (segment (start 143.5 111.58) (end 145.35 111.58) (width 1) (layer "F.Cu") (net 3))
 (segment (start 142.27 87.81) (end 139 91.08) (width 1) (layer "F.Cu") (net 3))
 (segment (start 121.81 110.65) (end 120.34 110.65) (width 1) (layer "F.Cu") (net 3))
 (segment (start 147 109.93) (end 147 101) (width 1) (layer "F.Cu") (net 3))
 (segment (start 114 110.5) (end 115.81 110.5) (width 1) (layer "F.Cu") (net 3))
 (segment (start 134.65 82.73) (end 142.27 82.73) (width 1) (layer "F.Cu") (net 3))
 (segment (start 147.5 96) (end 147.5 93.04) (width 1) (layer "F.Cu") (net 3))
 (segment (start 121.81 114.425585) (end 120.235585 116) (width 1) (layer "F.Cu") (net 3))
 (segment (start 139 92.92) (end 135.5 96.42) (width 1) (layer "F.Cu") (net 3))
 (segment (start 139 91.08) (end 139 92.92) (width 1) (layer "F.Cu") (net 3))
 (segment (start 142.825 64.5) (end 144.94632 64.5) (width 2) (layer "F.Cu") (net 3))
 (segment (start 147 101) (end 147 96.5) (width 1) (layer "F.Cu") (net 3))
 (segment (start 117.47 72.40868) (end 117.47 64.499415) (width 1) (layer "F.Cu") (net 3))
 (segment (start 110 111.5) (end 110 82.5) (width 1) (layer "F.Cu") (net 3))
 (segment (start 142.27 87.81) (end 147.35 92.89) (width 1) (layer "F.Cu") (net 3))
 (segment (start 147.5 93.04) (end 147.35 92.89) (width 1) (layer "F.Cu") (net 3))
 (segment (start 120.34 110.65) (end 118 108.31) (width 1) (layer "F.Cu") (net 3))
 (segment (start 115.81 110.5) (end 118 108.31) (width 1) (layer "F.Cu") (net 3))
 (segment (start 120.579415 61.39) (end 135.025 61.39) (width 1) (layer "F.Cu") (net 3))
 (segment (start 117.47 64.499415) (end 120.579415 61.39) (width 1) (layer "F.Cu") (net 3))
 (segment (start 129.43 95.41) (end 131.63 95.41) (width 1) (layer "F.Cu") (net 29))
 (segment (start 133.65 103.35) (end 136.794 103.35) (width 1) (layer "F.Cu") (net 29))
 (segment (start 136.794 103.35) (end 141.92 98.224) (width 1) (layer "F.Cu") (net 29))
 (segment (start 131.63 95.41) (end 131.63 101.33) (width 1) (layer "F.Cu") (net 29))
 (segment (start 141.92 98.224) (end 141.92 96.5) (width 1) (layer "F.Cu") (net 29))
 (segment (start 131.63 101.33) (end 133.65 103.35) (width 1) (layer "F.Cu") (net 29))
 (segment (start 111.5 106.717919) (end 111.5 110.616296) (width 1) (layer "F.Cu") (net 27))
 (segment (start 114 105.42) (end 112.797919 105.42) (width 1) (layer "F.Cu") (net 27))
 (segment (start 111.5 110.616296) (end 114.883704 114) (width 1) (layer "F.Cu") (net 27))
 (segment (start 112.797919 105.42) (end 111.5 106.717919) (width 1) (layer "F.Cu") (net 27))
 (segment (start 114.883704 114) (end 119.69 114) (width 1) (layer "F.Cu") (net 27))
 (segment (start 114.15 103.03) (end 114 102.88) (width 1) (layer "F.Cu") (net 38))
 (segment (start 121.81 103.03) (end 114.15 103.03) (width 1) (layer "F.Cu") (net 38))
 (segment (start 119.2 86.8) (end 118 88) (width 0.8) (layer "F.Cu") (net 33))
 (segment (start 119.2 85.055837) (end 119.2 86.8) (width 0.8) (layer "F.Cu") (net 33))
 (segment (start 118 96.34) (end 114 100.34) (width 0.8) (layer "F.Cu") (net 33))
 (segment (start 118 88) (end 118 96.34) (width 0.8) (layer "F.Cu") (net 33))
 (segment (start 121.81 82.71) (end 121.545837 82.71) (width 0.8) (layer "F.Cu") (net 33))
 (segment (start 121.545837 82.71) (end 119.2 85.055837) (width 0.8) (layer "F.Cu") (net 33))
 (segment (start 135.5 98.96) (end 134.46 98.96) (width 1) (layer "F.Cu") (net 7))
 (segment (start 133.5 94.74) (end 131.63 92.87) (width 1) (layer "F.Cu") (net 7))
 (segment (start 134.46 98.96) (end 133.5 98) (width 1) (layer "F.Cu") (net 7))
 (segment (start 133.5 98) (end 133.5 94.74) (width 1) (layer "F.Cu") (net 7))
 (segment (start 131.63 92.87) (end 129.43 92.87) (width 1) (layer "F.Cu") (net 7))
 (segment (start 152.78 82.73) (end 152.8 82.75) (width 1) (layer "F.Cu") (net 9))
 (segment (start 147.35 82.73) (end 152.78 82.73) (width 1) (layer "F.Cu") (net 9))
 (segment (start 152.8 87.75) (end 147.41 87.75) (width 1) (layer "F.Cu") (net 11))
 (segment (start 147.41 87.75) (end 147.35 87.81) (width 1) (layer "F.Cu") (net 11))
 (segment (start 152.78 85.27) (end 152.8 85.25) (width 1) (layer "F.Cu") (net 10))
 (segment (start 147.35 85.27) (end 152.78 85.27) (width 1) (layer "F.Cu") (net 10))
 (segment (start 147.35 80.19) (end 152.74 80.19) (width 1) (layer "F.Cu") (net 8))
 (segment (start 152.74 80.19) (end 152.8 80.25) (width 1) (layer "F.Cu") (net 8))
 (segment (start 131.7 108.11) (end 132.31 107.5) (width 1) (layer "F.Cu") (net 28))
 (segment (start 129.43 108.11) (end 131.7 108.11) (width 1) (layer "F.Cu") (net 28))
 (segment (start 121.61 100.69) (end 121.81 100.49) (width 1) (layer "F.Cu") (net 4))
 (segment (start 118 100.69) (end 121.61 100.69) (width 1) (layer "F.Cu") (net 4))
 (segment (start 132.896 83.104) (end 130.75 85.25) (width 1) (layer "F.Cu") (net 19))
 (segment (start 134.65 80.19) (end 132.896 81.944) (width 1) (layer "F.Cu") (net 19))
 (segment (start 132.896 81.944) (end 132.896 83.104) (width 1) (layer "F.Cu") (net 19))
 (segment (start 130.75 85.25) (end 129.43 85.25) (width 1) (layer "F.Cu") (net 19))
 (segment (start 129.43 82.71) (end 130.00868 82.71) (width 1) (layer "F.Cu") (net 20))
 (segment (start 132.896 79.404) (end 134.65 77.65) (width 1) (layer "F.Cu") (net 20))
 (segment (start 132.896 79.82268) (end 132.896 79.404) (width 1) (layer "F.Cu") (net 20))
 (segment (start 130.00868 82.71) (end 132.896 79.82268) (width 1) (layer "F.Cu") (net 20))
 (segment (start 132.09 87.79) (end 129.43 87.79) (width 1) (layer "F.Cu") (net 16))
 (segment (start 134.65 90.35) (end 132.09 87.79) (width 1) (layer "F.Cu") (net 16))
 (segment (start 117.6 76.420102) (end 117.6 82.978881) (width 0.8) (layer "F.Cu") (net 25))
 (segment (start 125.21 87.194163) (end 125.21 75.391522) (width 0.8) (layer "F.Cu") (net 25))
 (segment (start 122.074163 90.33) (end 125.21 87.194163) (width 0.8) (layer "F.Cu") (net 25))
 (segment (start 117.6 82.978881) (end 115.418881 85.16) (width 0.8) (layer "F.Cu") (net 25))
 (segment (start 115.202081 85.16) (end 114 85.16) (width 1) (layer "F.Cu") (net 25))
 (segment (start 119.590102 74.43) (end 117.6 76.420102) (width 0.8) (layer "F.Cu") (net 25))
 (segment (start 121.81 90.33) (end 122.074163 90.33) (width 0.8) (layer "F.Cu") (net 25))
 (segment (start 124.248478 74.43) (end 119.590102 74.43) (width 0.8) (layer "F.Cu") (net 25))
 (segment (start 125.21 75.391522) (end 124.248478 74.43) (width 0.8) (layer "F.Cu") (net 25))
 (segment (start 115.418881 85.16) (end 115.202081 85.16) (width 0.8) (layer "F.Cu") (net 25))
 (segment (start 132.896 76.864) (end 134.65 75.11) (width 1) (layer "F.Cu") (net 21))
 (segment (start 132.896 77.28268) (end 132.896 76.864) (width 1) (layer "F.Cu") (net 21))
 (segment (start 130.00868 80.17) (end 132.896 77.28268) (width 1) (layer "F.Cu") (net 21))
 (segment (start 129.43 80.17) (end 130.00868 80.17) (width 1) (layer "F.Cu") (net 21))
 (segment (start 132.09 90.33) (end 129.43 90.33) (width 1) (layer "F.Cu") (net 15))
 (segment (start 134.65 92.89) (end 132.09 90.33) (width 1) (layer "F.Cu") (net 15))
 (segment (start 128.43 105.57) (end 129.43 105.57) (width 1) (layer "F.Cu") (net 26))
 (segment (start 127 113.69) (end 127.31 114) (width 1) (layer "F.Cu") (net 26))
 (segment (start 129.024416 105.57) (end 127 107.594416) (width 1) (layer "F.Cu") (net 26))
 (segment (start 127 107.594416) (end 127 113.69) (width 1) (layer "F.Cu") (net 26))
 (segment (start 129.43 105.57) (end 129.024416 105.57) (width 1) (layer "F.Cu") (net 26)))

